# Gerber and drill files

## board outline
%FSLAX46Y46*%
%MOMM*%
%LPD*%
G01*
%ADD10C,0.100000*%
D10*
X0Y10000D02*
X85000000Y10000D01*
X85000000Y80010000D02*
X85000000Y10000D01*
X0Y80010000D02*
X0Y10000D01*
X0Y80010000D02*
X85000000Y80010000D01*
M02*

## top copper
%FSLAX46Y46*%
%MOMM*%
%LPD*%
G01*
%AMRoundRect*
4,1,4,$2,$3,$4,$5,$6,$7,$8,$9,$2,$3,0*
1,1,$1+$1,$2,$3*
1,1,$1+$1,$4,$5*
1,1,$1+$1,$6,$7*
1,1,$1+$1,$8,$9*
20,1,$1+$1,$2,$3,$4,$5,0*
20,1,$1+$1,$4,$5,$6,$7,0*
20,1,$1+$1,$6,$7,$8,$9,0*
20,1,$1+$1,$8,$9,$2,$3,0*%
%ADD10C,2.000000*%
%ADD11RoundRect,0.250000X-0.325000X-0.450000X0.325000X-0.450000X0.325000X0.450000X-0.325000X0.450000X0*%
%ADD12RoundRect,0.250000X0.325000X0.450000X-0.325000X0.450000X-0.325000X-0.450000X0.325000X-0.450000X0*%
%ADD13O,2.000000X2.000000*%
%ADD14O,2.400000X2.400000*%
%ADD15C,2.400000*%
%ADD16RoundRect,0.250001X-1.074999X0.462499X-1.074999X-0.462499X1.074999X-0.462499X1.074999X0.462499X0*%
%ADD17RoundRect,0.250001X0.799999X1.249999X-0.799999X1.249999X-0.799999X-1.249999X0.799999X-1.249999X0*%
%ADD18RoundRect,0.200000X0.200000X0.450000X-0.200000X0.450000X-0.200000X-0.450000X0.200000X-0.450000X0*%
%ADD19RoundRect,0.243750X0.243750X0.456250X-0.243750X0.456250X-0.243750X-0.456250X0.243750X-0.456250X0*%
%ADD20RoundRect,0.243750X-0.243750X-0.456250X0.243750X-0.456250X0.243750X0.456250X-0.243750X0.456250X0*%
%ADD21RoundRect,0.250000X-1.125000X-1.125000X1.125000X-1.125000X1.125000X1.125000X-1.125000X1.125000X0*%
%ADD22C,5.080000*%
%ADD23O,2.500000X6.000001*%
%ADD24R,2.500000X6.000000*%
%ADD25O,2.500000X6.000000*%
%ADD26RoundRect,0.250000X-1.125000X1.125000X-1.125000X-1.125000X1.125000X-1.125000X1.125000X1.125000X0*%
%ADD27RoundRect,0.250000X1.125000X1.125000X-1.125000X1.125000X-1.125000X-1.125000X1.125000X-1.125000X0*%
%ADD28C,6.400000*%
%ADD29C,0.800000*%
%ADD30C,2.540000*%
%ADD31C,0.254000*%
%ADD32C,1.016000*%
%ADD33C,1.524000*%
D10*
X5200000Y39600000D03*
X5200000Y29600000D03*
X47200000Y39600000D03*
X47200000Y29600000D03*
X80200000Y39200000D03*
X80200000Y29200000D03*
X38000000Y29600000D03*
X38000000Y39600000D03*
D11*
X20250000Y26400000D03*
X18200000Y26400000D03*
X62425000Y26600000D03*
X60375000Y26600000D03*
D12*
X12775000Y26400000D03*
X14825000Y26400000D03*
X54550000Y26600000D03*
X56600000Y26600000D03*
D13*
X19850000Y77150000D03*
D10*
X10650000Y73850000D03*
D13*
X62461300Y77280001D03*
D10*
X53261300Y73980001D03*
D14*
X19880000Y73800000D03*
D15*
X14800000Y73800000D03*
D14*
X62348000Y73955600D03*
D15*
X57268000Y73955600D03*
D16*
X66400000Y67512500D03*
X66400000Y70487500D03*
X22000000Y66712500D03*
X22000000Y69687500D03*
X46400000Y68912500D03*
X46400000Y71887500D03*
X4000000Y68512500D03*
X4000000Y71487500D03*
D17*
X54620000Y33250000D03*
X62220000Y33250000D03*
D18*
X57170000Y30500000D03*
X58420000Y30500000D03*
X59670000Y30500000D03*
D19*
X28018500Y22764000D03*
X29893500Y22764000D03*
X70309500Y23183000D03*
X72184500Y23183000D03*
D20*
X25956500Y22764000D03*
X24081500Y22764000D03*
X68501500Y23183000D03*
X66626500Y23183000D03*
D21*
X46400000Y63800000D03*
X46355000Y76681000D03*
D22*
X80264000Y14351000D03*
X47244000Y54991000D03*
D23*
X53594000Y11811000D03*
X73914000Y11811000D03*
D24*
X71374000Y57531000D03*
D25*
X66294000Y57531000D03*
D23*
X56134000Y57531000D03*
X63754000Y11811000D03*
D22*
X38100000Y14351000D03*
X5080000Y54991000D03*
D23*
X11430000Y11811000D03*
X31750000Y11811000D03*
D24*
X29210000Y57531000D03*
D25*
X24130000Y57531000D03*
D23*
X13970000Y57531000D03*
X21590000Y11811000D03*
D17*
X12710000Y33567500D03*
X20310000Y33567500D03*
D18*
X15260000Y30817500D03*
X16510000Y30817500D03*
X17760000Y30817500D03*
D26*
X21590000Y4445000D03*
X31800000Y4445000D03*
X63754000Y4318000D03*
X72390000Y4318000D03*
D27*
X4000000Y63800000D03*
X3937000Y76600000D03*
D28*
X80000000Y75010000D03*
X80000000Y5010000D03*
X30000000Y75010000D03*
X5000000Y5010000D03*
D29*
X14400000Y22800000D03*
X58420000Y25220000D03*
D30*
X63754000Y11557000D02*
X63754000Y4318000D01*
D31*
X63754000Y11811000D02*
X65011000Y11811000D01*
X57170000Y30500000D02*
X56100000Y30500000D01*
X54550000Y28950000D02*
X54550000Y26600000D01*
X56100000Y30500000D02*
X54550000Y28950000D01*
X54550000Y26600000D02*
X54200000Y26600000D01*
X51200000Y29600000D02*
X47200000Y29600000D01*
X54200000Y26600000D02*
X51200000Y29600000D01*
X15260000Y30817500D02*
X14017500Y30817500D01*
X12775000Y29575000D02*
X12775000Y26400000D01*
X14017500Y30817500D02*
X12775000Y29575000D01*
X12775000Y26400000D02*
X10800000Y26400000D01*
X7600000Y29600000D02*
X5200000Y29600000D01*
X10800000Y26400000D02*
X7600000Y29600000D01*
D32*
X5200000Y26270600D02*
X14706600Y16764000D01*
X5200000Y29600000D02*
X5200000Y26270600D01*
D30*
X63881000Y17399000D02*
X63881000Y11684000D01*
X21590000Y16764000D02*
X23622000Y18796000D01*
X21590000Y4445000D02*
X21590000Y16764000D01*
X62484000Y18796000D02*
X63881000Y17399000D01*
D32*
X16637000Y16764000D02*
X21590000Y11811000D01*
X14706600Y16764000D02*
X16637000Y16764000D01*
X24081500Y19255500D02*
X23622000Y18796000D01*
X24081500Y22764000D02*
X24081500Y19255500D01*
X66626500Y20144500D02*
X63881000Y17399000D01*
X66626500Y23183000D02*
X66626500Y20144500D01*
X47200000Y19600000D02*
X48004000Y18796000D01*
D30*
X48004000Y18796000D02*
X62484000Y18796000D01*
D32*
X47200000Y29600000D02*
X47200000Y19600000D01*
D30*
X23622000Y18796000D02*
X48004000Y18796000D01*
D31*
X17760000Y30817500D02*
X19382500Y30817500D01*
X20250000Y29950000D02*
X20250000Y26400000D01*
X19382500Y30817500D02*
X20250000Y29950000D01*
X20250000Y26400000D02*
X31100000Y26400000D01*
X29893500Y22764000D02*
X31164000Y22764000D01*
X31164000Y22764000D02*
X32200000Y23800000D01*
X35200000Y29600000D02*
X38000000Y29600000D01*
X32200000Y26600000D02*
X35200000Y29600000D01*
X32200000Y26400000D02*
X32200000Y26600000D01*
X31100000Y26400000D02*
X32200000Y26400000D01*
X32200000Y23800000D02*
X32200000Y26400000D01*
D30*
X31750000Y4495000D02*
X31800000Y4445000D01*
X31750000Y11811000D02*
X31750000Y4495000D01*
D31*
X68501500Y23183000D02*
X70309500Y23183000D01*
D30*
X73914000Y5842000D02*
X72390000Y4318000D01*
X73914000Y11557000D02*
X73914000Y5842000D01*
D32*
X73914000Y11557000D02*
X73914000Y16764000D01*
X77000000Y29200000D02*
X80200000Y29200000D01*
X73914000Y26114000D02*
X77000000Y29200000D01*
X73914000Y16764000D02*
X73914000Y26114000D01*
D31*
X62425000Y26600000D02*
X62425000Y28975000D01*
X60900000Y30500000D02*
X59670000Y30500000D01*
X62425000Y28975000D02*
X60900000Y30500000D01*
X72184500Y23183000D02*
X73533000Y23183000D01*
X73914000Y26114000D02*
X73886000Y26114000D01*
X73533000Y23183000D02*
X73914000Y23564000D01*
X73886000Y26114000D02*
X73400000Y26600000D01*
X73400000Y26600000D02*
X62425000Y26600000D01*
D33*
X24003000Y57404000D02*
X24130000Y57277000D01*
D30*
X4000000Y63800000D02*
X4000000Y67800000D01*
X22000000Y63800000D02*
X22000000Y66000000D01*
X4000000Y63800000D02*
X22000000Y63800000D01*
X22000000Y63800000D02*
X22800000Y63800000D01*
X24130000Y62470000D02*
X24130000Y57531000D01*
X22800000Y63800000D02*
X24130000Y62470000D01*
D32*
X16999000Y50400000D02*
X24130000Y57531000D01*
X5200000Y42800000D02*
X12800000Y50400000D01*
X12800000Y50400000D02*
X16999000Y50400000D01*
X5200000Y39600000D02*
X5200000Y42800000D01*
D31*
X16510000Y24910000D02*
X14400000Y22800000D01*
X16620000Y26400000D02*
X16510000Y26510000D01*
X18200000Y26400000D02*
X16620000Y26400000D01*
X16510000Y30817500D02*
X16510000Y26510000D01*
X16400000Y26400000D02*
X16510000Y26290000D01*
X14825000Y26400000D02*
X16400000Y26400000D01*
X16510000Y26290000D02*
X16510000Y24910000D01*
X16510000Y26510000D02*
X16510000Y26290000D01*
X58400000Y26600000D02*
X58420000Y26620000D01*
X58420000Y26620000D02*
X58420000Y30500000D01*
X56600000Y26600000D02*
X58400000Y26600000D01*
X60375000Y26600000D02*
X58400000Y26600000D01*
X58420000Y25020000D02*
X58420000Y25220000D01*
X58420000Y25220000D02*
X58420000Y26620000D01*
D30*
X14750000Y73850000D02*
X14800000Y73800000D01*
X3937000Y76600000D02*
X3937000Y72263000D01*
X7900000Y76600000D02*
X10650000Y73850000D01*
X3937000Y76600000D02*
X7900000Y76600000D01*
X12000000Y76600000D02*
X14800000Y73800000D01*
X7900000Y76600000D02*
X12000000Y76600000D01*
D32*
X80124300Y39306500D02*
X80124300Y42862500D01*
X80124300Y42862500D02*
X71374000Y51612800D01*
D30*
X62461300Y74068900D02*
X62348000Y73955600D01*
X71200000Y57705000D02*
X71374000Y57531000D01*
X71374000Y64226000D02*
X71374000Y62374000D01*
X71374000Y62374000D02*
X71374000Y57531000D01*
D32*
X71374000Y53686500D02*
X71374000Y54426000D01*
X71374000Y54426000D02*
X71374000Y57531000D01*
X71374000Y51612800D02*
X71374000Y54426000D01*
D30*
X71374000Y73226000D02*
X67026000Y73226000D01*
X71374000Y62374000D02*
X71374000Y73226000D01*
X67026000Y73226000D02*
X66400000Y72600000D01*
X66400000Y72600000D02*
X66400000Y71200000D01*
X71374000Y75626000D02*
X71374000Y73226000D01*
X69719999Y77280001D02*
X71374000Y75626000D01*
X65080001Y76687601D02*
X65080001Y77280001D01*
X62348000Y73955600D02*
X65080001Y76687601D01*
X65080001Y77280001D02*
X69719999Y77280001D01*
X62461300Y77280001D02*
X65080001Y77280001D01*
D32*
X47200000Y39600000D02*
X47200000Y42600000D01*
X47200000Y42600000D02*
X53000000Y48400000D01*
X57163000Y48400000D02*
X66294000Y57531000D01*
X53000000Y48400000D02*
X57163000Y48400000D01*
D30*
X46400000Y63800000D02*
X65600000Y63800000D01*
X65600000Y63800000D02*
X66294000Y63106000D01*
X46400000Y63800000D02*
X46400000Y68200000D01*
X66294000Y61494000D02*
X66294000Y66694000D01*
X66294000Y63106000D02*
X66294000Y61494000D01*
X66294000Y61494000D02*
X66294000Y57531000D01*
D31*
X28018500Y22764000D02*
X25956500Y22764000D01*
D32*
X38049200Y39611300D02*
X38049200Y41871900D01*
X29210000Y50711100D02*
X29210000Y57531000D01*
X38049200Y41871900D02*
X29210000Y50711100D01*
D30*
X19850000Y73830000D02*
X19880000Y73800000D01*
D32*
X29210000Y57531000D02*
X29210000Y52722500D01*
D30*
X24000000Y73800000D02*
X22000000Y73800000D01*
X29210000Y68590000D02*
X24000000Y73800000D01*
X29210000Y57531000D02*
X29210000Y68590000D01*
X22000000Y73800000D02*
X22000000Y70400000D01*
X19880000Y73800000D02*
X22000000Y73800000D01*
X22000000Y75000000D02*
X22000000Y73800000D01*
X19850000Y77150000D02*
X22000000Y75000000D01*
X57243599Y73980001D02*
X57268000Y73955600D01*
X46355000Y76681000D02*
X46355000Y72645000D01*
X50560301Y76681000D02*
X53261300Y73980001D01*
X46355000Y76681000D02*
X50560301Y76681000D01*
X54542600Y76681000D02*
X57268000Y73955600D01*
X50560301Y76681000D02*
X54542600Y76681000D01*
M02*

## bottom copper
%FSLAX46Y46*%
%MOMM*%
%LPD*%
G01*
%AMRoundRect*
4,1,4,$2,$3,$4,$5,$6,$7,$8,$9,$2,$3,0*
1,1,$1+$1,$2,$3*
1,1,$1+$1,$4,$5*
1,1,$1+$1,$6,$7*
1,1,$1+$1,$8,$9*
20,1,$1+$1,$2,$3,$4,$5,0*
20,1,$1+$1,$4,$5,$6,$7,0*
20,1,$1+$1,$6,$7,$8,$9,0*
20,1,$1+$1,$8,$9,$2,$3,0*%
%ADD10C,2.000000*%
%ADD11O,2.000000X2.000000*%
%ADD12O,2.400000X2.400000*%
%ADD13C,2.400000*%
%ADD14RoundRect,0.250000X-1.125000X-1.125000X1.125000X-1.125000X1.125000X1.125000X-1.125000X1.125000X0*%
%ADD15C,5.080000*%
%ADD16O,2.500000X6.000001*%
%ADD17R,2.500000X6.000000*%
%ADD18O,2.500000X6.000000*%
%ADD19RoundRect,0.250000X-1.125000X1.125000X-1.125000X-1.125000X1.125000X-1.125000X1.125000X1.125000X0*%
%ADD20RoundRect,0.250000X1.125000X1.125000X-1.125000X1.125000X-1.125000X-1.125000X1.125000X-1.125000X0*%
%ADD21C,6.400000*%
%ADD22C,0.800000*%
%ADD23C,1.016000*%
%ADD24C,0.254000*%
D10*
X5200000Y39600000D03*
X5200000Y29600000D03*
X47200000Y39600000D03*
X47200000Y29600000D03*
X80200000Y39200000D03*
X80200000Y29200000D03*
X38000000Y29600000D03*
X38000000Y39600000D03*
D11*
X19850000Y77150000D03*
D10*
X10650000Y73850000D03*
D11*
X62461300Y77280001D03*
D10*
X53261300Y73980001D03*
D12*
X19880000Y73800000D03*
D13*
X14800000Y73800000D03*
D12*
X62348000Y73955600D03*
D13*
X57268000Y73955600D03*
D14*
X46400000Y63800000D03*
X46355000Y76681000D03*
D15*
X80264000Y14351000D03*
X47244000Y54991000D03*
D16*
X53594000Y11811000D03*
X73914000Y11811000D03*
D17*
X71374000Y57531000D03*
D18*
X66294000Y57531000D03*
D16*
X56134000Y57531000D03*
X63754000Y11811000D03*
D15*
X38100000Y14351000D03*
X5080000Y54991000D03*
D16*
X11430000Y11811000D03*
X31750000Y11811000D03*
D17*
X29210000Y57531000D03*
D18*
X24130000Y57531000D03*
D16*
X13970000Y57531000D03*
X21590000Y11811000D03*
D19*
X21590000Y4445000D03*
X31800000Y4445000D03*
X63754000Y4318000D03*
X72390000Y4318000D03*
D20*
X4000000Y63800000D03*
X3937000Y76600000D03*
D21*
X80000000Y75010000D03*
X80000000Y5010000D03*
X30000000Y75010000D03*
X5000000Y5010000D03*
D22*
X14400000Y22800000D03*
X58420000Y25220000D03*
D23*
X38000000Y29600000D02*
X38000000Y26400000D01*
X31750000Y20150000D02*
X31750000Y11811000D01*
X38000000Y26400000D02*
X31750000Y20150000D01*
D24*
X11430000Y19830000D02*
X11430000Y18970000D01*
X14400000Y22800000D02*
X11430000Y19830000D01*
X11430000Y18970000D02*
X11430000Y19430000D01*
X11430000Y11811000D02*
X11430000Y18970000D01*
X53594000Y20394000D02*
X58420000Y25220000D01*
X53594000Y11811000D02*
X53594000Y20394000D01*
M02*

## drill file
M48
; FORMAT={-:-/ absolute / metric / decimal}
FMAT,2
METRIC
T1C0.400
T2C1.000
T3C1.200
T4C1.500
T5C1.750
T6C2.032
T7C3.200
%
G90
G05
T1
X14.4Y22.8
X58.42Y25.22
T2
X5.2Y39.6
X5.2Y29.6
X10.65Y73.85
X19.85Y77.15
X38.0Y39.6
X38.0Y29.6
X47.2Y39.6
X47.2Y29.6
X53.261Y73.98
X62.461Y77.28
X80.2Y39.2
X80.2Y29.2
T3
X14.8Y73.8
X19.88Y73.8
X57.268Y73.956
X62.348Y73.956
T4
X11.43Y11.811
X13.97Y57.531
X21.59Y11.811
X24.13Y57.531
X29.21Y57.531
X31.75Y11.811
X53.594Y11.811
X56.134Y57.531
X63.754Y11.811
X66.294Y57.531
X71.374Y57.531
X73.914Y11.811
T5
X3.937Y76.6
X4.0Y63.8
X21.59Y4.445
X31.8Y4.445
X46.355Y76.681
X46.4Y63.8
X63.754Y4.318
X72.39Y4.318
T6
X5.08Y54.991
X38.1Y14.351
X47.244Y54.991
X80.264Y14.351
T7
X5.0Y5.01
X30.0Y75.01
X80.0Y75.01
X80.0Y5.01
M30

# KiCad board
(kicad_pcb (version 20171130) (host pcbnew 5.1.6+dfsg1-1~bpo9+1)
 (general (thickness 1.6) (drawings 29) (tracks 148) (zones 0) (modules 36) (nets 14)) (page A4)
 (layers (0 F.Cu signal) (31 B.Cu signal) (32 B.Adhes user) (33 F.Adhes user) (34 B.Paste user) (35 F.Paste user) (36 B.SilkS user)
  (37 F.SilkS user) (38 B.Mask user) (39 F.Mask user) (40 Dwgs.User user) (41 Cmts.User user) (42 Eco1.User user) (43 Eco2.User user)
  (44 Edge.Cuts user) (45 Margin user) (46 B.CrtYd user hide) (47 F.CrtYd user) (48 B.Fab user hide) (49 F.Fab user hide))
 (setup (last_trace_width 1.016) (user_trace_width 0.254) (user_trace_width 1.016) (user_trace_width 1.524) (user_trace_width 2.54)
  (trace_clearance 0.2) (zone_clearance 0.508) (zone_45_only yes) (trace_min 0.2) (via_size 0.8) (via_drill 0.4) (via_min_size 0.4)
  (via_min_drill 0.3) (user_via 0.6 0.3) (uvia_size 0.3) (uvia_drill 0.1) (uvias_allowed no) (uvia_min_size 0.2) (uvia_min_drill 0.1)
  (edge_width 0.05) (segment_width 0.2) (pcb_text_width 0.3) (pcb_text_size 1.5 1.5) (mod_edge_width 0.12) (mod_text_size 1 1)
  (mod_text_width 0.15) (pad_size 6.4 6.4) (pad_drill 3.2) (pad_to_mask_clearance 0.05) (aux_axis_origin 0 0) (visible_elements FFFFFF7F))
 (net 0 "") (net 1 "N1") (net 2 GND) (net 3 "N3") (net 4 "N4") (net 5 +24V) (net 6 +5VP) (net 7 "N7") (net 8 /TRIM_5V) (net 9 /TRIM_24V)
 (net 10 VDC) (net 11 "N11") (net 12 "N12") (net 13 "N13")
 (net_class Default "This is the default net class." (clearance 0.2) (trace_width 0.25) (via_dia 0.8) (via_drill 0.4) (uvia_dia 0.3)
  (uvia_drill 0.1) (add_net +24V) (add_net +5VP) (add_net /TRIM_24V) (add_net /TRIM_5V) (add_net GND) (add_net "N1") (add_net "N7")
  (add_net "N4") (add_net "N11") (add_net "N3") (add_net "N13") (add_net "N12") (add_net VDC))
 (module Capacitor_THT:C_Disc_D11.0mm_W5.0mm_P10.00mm (layer F.Cu) (at 5.2 -29.6 90)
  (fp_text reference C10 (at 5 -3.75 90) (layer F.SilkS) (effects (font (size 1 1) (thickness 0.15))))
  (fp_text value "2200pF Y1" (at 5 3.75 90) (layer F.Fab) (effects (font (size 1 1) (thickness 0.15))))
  (pad 2 thru_hole circle (at 10 0 90) (size 2 2) (drill 1) (layers *.Cu *.Mask) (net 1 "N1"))
  (pad 1 thru_hole circle (at 0 0 90) (size 2 2) (drill 1) (layers *.Cu *.Mask) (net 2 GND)))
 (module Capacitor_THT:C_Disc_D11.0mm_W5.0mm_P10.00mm (layer F.Cu) (at 47.2 -29.6 90)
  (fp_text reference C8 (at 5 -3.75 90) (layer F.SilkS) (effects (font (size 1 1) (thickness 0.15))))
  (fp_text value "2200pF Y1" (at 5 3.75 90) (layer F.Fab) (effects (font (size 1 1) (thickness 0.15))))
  (pad 2 thru_hole circle (at 10 0 90) (size 2 2) (drill 1) (layers *.Cu *.Mask) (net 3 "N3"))
  (pad 1 thru_hole circle (at 0 0 90) (size 2 2) (drill 1) (layers *.Cu *.Mask) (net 2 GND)))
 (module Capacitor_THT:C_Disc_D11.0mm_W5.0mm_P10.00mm (layer F.Cu) (at 80.2 -29.2 90)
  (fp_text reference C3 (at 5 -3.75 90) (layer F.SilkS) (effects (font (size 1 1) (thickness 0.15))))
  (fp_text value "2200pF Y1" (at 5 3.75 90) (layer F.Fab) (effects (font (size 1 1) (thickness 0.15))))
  (pad 2 thru_hole circle (at 10 0 90) (size 2 2) (drill 1) (layers *.Cu *.Mask) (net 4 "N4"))
  (pad 1 thru_hole circle (at 0 0 90) (size 2 2) (drill 1) (layers *.Cu *.Mask) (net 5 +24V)))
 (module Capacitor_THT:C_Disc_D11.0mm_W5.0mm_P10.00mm (layer F.Cu) (at 38 -39.6 270)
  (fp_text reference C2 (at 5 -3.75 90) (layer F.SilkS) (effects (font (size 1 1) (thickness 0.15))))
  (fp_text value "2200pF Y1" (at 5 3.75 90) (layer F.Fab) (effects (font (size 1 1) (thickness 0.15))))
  (pad 2 thru_hole circle (at 10 0 270) (size 2 2) (drill 1) (layers *.Cu *.Mask) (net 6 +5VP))
  (pad 1 thru_hole circle (at 0 0 270) (size 2 2) (drill 1) (layers *.Cu *.Mask) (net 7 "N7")))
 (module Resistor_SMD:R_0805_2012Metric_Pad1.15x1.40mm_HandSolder (layer F.Cu) (at 19.225 -26.4)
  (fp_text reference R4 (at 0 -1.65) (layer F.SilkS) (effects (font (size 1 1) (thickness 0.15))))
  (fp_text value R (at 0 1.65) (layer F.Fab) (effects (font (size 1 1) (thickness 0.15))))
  (pad 2 smd roundrect (at 1.025 0) (size 1.15 1.4) (layers F.Cu F.Paste F.Mask) (roundrect_rratio 0.217391) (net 6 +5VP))
  (pad 1 smd roundrect (at -1.025 0) (size 1.15 1.4) (layers F.Cu F.Paste F.Mask) (roundrect_rratio 0.217391) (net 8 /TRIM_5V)))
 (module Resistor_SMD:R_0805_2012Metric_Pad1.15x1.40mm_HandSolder (layer F.Cu) (at 61.4 -26.6)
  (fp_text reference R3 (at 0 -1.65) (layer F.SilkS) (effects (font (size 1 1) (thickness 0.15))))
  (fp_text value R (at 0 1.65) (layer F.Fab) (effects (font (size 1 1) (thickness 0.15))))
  (pad 2 smd roundrect (at 1.025 0) (size 1.15 1.4) (layers F.Cu F.Paste F.Mask) (roundrect_rratio 0.217391) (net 5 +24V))
  (pad 1 smd roundrect (at -1.025 0) (size 1.15 1.4) (layers F.Cu F.Paste F.Mask) (roundrect_rratio 0.217391) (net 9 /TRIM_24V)))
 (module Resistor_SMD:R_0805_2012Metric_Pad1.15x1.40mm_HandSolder (layer F.Cu) (at 13.8 -26.4 180)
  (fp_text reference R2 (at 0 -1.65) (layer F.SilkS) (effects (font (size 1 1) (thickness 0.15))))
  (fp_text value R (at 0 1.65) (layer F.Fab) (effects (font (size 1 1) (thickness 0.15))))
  (pad 2 smd roundrect (at 1.025 0 180) (size 1.15 1.4) (layers F.Cu F.Paste F.Mask) (roundrect_rratio 0.217391) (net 2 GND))
  (pad 1 smd roundrect (at -1.025 0 180) (size 1.15 1.4) (layers F.Cu F.Paste F.Mask) (roundrect_rratio 0.217391) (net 8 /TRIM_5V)))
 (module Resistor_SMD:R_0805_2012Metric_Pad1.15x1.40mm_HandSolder (layer F.Cu) (at 55.575 -26.6 180)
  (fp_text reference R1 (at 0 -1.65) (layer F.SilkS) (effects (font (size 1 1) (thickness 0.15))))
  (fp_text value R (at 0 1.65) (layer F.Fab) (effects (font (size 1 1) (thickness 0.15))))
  (pad 2 smd roundrect (at 1.025 0 180) (size 1.15 1.4) (layers F.Cu F.Paste F.Mask) (roundrect_rratio 0.217391) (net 2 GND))
  (pad 1 smd roundrect (at -1.025 0 180) (size 1.15 1.4) (layers F.Cu F.Paste F.Mask) (roundrect_rratio 0.217391) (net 9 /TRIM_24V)))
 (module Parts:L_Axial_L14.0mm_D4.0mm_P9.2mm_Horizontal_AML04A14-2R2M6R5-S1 (layer F.Cu) (at 10.65 -73.85)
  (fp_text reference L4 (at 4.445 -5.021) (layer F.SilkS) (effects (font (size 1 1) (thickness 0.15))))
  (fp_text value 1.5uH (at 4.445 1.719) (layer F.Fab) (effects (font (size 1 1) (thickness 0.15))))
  (pad 2 thru_hole oval (at 9.2 -3.3) (size 2 2) (drill 1) (layers *.Cu *.Mask) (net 7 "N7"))
  (pad 1 thru_hole circle (at 0 0) (size 2 2) (drill 1) (layers *.Cu *.Mask) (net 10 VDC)))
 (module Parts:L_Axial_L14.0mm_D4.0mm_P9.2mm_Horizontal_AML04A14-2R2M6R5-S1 (layer F.Cu) (at 53.2613 -73.980001)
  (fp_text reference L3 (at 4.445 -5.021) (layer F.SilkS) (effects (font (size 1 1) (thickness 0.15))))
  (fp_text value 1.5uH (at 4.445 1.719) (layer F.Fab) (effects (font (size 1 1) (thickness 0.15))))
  (pad 2 thru_hole oval (at 9.2 -3.3) (size 2 2) (drill 1) (layers *.Cu *.Mask) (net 4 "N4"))
  (pad 1 thru_hole circle (at 0 0) (size 2 2) (drill 1) (layers *.Cu *.Mask) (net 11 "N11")))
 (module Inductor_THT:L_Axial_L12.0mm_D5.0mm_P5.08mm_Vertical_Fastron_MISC (layer F.Cu) (at 14.8 -73.8)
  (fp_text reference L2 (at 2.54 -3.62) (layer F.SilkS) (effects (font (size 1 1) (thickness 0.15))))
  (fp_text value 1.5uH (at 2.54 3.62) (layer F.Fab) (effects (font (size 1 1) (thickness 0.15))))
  (pad 2 thru_hole oval (at 5.08 0) (size 2.4 2.4) (drill 1.2) (layers *.Cu *.Mask) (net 7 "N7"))
  (pad 1 thru_hole circle (at 0 0) (size 2.4 2.4) (drill 1.2) (layers *.Cu *.Mask) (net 10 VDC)))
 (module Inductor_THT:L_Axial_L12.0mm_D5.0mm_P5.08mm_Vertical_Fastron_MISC (layer F.Cu) (at 57.268 -73.9556)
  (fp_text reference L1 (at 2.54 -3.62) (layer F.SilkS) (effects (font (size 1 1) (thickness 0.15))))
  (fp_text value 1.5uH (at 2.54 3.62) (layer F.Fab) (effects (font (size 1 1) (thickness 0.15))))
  (pad 2 thru_hole oval (at 5.08 0) (size 2.4 2.4) (drill 1.2) (layers *.Cu *.Mask) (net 4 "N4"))
  (pad 1 thru_hole circle (at 0 0) (size 2.4 2.4) (drill 1.2) (layers *.Cu *.Mask) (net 11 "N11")))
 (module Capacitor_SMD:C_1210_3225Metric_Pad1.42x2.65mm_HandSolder (layer F.Cu) (at 66.4 -69 270)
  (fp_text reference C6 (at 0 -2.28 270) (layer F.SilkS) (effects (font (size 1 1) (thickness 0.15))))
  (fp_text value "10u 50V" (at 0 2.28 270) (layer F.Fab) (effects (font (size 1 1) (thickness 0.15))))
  (pad 2 smd roundrect (at 1.4875 0 270) (size 1.425 2.65) (layers F.Cu F.Paste F.Mask) (roundrect_rratio 0.175439) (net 3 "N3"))
  (pad 1 smd roundrect (at -1.4875 0 270) (size 1.425 2.65) (layers F.Cu F.Paste F.Mask) (roundrect_rratio 0.175439) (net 4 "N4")))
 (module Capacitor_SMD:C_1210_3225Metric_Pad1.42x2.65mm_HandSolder (layer F.Cu) (at 22 -68.2 270)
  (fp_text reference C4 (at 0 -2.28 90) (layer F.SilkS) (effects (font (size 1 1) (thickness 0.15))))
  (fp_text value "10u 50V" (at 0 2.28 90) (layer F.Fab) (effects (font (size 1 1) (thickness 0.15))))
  (pad 2 smd roundrect (at 1.4875 0 270) (size 1.425 2.65) (layers F.Cu F.Paste F.Mask) (roundrect_rratio 0.175439) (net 1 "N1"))
  (pad 1 smd roundrect (at -1.4875 0 270) (size 1.425 2.65) (layers F.Cu F.Paste F.Mask) (roundrect_rratio 0.175439) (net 7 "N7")))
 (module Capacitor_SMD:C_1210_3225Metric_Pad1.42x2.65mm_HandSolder (layer F.Cu) (at 46.4 -70.4 270)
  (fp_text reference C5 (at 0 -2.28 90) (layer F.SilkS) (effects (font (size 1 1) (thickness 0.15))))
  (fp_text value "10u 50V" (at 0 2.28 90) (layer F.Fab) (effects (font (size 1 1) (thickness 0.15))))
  (pad 2 smd roundrect (at 1.4875 0 270) (size 1.425 2.65) (layers F.Cu F.Paste F.Mask) (roundrect_rratio 0.175439) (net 3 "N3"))
  (pad 1 smd roundrect (at -1.4875 0 270) (size 1.425 2.65) (layers F.Cu F.Paste F.Mask) (roundrect_rratio 0.175439) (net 11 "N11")))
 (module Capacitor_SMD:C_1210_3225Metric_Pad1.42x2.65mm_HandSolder (layer F.Cu) (at 4 -70 270)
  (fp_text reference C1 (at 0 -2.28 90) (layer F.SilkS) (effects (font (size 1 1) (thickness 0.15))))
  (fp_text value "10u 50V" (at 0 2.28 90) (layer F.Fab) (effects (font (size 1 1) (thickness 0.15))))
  (pad 2 smd roundrect (at 1.4875 0 270) (size 1.425 2.65) (layers F.Cu F.Paste F.Mask) (roundrect_rratio 0.175439) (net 1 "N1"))
  (pad 1 smd roundrect (at -1.4875 0 270) (size 1.425 2.65) (layers F.Cu F.Paste F.Mask) (roundrect_rratio 0.175439) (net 10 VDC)))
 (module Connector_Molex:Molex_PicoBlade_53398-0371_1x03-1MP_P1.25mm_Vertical (layer F.Cu) (at 58.42 -31.75 180)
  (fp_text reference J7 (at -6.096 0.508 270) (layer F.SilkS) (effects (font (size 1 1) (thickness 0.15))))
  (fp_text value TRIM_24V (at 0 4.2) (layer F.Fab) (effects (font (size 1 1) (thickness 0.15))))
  (pad MP smd roundrect (at 3.8 1.5 180) (size 2.1 3) (layers F.Cu F.Paste F.Mask) (roundrect_rratio 0.119048))
  (pad MP smd roundrect (at -3.8 1.5 180) (size 2.1 3) (layers F.Cu F.Paste F.Mask) (roundrect_rratio 0.119048))
  (pad 3 smd roundrect (at 1.25 -1.25 180) (size 0.8 1.3) (layers F.Cu F.Paste F.Mask) (roundrect_rratio 0.25) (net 2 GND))
  (pad 2 smd roundrect (at 0 -1.25 180) (size 0.8 1.3) (layers F.Cu F.Paste F.Mask) (roundrect_rratio 0.25) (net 9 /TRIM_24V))
  (pad 1 smd roundrect (at -1.25 -1.25 180) (size 0.8 1.3) (layers F.Cu F.Paste F.Mask) (roundrect_rratio 0.25) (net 5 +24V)))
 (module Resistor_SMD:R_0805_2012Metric (layer F.Cu) (at 28.956 -22.764 180)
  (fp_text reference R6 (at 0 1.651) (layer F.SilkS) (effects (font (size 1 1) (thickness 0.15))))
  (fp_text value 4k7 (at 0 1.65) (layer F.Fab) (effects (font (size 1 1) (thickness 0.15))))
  (pad 2 smd roundrect (at 0.9375 0 180) (size 0.975 1.4) (layers F.Cu F.Paste F.Mask) (roundrect_rratio 0.25) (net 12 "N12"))
  (pad 1 smd roundrect (at -0.9375 0 180) (size 0.975 1.4) (layers F.Cu F.Paste F.Mask) (roundrect_rratio 0.25) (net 6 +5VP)))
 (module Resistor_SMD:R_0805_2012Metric (layer F.Cu) (at 71.247 -23.183 180)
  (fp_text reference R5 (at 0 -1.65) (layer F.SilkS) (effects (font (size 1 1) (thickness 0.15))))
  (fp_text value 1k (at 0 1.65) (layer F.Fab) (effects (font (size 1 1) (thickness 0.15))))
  (pad 2 smd roundrect (at 0.9375 0 180) (size 0.975 1.4) (layers F.Cu F.Paste F.Mask) (roundrect_rratio 0.25) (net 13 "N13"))
  (pad 1 smd roundrect (at -0.9375 0 180) (size 0.975 1.4) (layers F.Cu F.Paste F.Mask) (roundrect_rratio 0.25) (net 5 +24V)))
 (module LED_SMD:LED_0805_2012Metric (layer F.Cu) (at 25.019 -22.764)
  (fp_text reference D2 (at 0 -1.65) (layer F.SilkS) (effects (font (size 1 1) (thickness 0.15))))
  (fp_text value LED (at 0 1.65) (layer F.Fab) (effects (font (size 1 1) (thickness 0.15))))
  (pad 2 smd roundrect (at 0.9375 0) (size 0.975 1.4) (layers F.Cu F.Paste F.Mask) (roundrect_rratio 0.25) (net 12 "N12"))
  (pad 1 smd roundrect (at -0.9375 0) (size 0.975 1.4) (layers F.Cu F.Paste F.Mask) (roundrect_rratio 0.25) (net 2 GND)))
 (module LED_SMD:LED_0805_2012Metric (layer F.Cu) (at 67.564 -23.183)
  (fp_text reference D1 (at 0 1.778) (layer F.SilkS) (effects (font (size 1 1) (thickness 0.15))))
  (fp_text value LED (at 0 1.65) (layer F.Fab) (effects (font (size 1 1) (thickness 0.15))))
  (pad 2 smd roundrect (at 0.9375 0) (size 0.975 1.4) (layers F.Cu F.Paste F.Mask) (roundrect_rratio 0.25) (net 13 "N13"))
  (pad 1 smd roundrect (at -0.9375 0) (size 0.975 1.4) (layers F.Cu F.Paste F.Mask) (roundrect_rratio 0.25) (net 2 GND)))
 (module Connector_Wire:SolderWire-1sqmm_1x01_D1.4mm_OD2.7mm (layer F.Cu) (at 46.4 -63.8)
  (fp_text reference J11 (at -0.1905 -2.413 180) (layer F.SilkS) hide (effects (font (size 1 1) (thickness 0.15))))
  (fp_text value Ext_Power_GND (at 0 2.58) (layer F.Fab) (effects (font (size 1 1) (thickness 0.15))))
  (pad 1 thru_hole roundrect (at 0 0) (size 2.75 2.75) (drill 1.75) (layers *.Cu *.Mask) (roundrect_rratio 0.090909) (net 3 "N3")))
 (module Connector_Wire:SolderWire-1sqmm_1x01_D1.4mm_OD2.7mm (layer F.Cu) (at 46.355 -76.681)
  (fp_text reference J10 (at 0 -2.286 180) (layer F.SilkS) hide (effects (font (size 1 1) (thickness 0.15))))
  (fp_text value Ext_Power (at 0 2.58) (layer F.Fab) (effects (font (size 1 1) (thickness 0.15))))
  (pad 1 thru_hole roundrect (at 0 0) (size 2.75 2.75) (drill 1.75) (layers *.Cu *.Mask) (roundrect_rratio 0.090909) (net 11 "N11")))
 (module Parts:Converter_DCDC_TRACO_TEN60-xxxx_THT (layer B.Cu) (at 71.374 -57.531 180)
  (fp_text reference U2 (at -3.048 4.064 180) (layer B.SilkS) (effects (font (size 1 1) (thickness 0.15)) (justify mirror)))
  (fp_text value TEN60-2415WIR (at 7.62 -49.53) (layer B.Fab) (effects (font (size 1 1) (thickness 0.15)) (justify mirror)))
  (pad 8 thru_hole circle (at -8.89 -43.18 90) (size 5.08 5.08) (drill 2.032) (layers *.Cu *.Mask))
  (pad 7 thru_hole circle (at 24.13 -2.54 90) (size 5.08 5.08) (drill 2.032) (layers *.Cu *.Mask))
  (pad 6 thru_hole oval (at 17.78 -45.72 90) (size 6.000001 2.5) (drill 1.5) (layers *.Cu *.Mask) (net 9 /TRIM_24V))
  (pad 4 thru_hole oval (at -2.54 -45.72 90) (size 6.000001 2.5) (drill 1.5) (layers *.Cu *.Mask) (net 5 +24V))
  (pad 1 thru_hole rect (at 0 0 90) (size 6 2.5) (drill 1.5) (layers *.Cu *.Mask) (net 4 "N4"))
  (pad 2 thru_hole oval (at 5.08 0 90) (size 6 2.5) (drill 1.5) (layers *.Cu *.Mask) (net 3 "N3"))
  (pad 3 thru_hole oval (at 15.24 0 90) (size 6.000001 2.5) (drill 1.5) (layers *.Cu *.Mask))
  (pad 5 thru_hole oval (at 7.62 -45.72 90) (size 6.000001 2.5) (drill 1.5) (layers *.Cu *.Mask) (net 2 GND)))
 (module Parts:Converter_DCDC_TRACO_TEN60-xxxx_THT (layer B.Cu) (at 29.21 -57.531 180)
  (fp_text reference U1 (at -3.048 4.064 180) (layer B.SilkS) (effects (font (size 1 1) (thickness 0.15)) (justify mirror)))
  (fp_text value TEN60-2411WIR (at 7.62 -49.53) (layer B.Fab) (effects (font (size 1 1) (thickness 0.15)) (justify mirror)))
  (pad 8 thru_hole circle (at -8.89 -43.18 90) (size 5.08 5.08) (drill 2.032) (layers *.Cu *.Mask))
  (pad 7 thru_hole circle (at 24.13 -2.54 90) (size 5.08 5.08) (drill 2.032) (layers *.Cu *.Mask))
  (pad 6 thru_hole oval (at 17.78 -45.72 90) (size 6.000001 2.5) (drill 1.5) (layers *.Cu *.Mask) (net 8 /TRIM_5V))
  (pad 4 thru_hole oval (at -2.54 -45.72 90) (size 6.000001 2.5) (drill 1.5) (layers *.Cu *.Mask) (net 6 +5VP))
  (pad 1 thru_hole rect (at 0 0 90) (size 6 2.5) (drill 1.5) (layers *.Cu *.Mask) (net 7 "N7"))
  (pad 2 thru_hole oval (at 5.08 0 90) (size 6 2.5) (drill 1.5) (layers *.Cu *.Mask) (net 1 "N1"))
  (pad 3 thru_hole oval (at 15.24 0 90) (size 6.000001 2.5) (drill 1.5) (layers *.Cu *.Mask))
  (pad 5 thru_hole oval (at 7.62 -45.72 90) (size 6.000001 2.5) (drill 1.5) (layers *.Cu *.Mask) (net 2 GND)))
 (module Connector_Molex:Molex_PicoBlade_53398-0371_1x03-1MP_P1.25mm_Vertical (layer F.Cu) (at 16.51 -32.0675 180)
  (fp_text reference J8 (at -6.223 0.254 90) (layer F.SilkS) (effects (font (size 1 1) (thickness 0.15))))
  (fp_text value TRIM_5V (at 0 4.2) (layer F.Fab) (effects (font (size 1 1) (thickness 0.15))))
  (pad MP smd roundrect (at 3.8 1.5 180) (size 2.1 3) (layers F.Cu F.Paste F.Mask) (roundrect_rratio 0.119048))
  (pad MP smd roundrect (at -3.8 1.5 180) (size 2.1 3) (layers F.Cu F.Paste F.Mask) (roundrect_rratio 0.119048))
  (pad 3 smd roundrect (at 1.25 -1.25 180) (size 0.8 1.3) (layers F.Cu F.Paste F.Mask) (roundrect_rratio 0.25) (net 2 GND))
  (pad 2 smd roundrect (at 0 -1.25 180) (size 0.8 1.3) (layers F.Cu F.Paste F.Mask) (roundrect_rratio 0.25) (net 8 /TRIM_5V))
  (pad 1 smd roundrect (at -1.25 -1.25 180) (size 0.8 1.3) (layers F.Cu F.Paste F.Mask) (roundrect_rratio 0.25) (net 6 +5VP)))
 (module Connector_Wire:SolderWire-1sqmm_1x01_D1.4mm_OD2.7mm (layer F.Cu) (at 21.59 -4.445 270)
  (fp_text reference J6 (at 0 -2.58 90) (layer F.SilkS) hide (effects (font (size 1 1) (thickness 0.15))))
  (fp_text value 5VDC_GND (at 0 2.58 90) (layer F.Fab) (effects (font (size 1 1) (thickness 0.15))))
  (pad 1 thru_hole roundrect (at 0 0 270) (size 2.75 2.75) (drill 1.75) (layers *.Cu *.Mask) (roundrect_rratio 0.090909) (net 2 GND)))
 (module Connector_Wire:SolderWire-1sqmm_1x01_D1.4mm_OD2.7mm (layer F.Cu) (at 31.8 -4.445 270)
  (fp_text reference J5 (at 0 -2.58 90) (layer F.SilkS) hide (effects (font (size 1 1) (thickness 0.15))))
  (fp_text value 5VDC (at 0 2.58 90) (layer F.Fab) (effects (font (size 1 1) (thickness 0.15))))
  (pad 1 thru_hole roundrect (at 0 0 270) (size 2.75 2.75) (drill 1.75) (layers *.Cu *.Mask) (roundrect_rratio 0.090909) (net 6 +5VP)))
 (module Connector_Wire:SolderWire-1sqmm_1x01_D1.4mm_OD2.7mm (layer F.Cu) (at 63.754 -4.318 270)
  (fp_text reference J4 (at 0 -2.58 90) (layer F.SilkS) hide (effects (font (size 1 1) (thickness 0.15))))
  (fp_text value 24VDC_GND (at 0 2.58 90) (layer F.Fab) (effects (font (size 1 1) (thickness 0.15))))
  (pad 1 thru_hole roundrect (at 0 0 270) (size 2.75 2.75) (drill 1.75) (layers *.Cu *.Mask) (roundrect_rratio 0.090909) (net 2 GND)))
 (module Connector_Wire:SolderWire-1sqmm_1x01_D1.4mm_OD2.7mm (layer F.Cu) (at 72.39 -4.318 270)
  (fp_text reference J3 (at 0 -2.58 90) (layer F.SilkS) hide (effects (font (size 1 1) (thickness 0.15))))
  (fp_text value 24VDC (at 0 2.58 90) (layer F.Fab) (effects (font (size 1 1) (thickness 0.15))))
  (pad 1 thru_hole roundrect (at 0 0 270) (size 2.75 2.75) (drill 1.75) (layers *.Cu *.Mask) (roundrect_rratio 0.090909) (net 5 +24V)))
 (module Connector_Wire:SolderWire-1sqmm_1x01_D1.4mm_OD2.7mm (layer F.Cu) (at 4 -63.8 180)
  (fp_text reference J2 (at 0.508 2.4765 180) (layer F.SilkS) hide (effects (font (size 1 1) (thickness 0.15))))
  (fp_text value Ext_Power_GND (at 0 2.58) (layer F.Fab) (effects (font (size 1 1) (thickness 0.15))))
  (pad 1 thru_hole roundrect (at 0 0 180) (size 2.75 2.75) (drill 1.75) (layers *.Cu *.Mask) (roundrect_rratio 0.090909) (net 1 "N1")))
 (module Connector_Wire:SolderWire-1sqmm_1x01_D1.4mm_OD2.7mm (layer F.Cu) (at 3.937 -76.6 180)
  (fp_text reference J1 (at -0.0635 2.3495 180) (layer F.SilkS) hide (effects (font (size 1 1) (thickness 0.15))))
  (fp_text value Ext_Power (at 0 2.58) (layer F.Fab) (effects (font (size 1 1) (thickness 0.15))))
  (pad 1 thru_hole roundrect (at 0 0 180) (size 2.75 2.75) (drill 1.75) (layers *.Cu *.Mask) (roundrect_rratio 0.090909) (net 10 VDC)))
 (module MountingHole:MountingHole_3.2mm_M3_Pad (layer F.Cu) (at 80 -75.01)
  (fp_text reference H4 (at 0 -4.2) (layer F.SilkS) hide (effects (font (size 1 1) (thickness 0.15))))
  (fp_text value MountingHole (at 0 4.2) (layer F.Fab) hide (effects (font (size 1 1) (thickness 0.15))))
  (pad 1 thru_hole circle (at 0 0) (size 6.4 6.4) (drill 3.2) (layers *.Cu *.Mask)))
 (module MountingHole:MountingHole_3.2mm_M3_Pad (layer F.Cu) (at 80 -5.01)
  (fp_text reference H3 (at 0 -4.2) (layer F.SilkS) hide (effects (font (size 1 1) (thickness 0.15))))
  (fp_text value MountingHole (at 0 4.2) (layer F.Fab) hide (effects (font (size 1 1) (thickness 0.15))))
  (pad 1 thru_hole circle (at 0 0) (size 6.4 6.4) (drill 3.2) (layers *.Cu *.Mask)))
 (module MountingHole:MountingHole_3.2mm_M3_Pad (layer F.Cu) (at 30 -75.01)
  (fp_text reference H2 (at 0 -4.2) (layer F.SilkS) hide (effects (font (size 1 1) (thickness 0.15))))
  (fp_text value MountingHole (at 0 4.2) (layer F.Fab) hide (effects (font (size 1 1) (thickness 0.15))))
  (pad 1 thru_hole circle (at 0 0) (size 6.4 6.4) (drill 3.2) (layers *.Cu *.Mask)))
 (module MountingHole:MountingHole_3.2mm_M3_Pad (layer F.Cu) (at 5 -5.01)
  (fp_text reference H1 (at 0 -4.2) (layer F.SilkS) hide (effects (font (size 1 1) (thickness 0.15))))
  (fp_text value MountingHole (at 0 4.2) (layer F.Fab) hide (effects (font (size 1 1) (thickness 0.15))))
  (pad 1 thru_hole circle (at 0 0) (size 6.4 6.4) (drill 3.2) (layers *.Cu *.Mask)))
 (gr_line (start 0 -0.01) (end 85 -0.01) (layer Edge.Cuts) (width 0.1))
 (gr_line (start 85 -80.01) (end 85 -0.01) (layer Edge.Cuts) (width 0.1))
 (gr_line (start 0 -80.01) (end 0 -0.01) (layer Edge.Cuts) (width 0.1))
 (gr_line (start 0 -80.01) (end 85 -80.01) (layer Edge.Cuts) (width 0.1))
 (segment (start 63.754 -11.557) (end 63.754 -4.318) (width 2.54) (layer F.Cu) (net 2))
 (segment (start 63.754 -11.811) (end 65.011 -11.811) (width 0.254) (layer F.Cu) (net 2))
 (segment (start 57.17 -30.5) (end 56.1 -30.5) (width 0.254) (layer F.Cu) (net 2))
 (segment (start 54.55 -28.95) (end 54.55 -26.6) (width 0.254) (layer F.Cu) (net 2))
 (segment (start 56.1 -30.5) (end 54.55 -28.95) (width 0.254) (layer F.Cu) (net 2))
 (segment (start 54.55 -26.6) (end 54.2 -26.6) (width 0.254) (layer F.Cu) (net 2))
 (segment (start 51.2 -29.6) (end 47.2 -29.6) (width 0.254) (layer F.Cu) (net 2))
 (segment (start 54.2 -26.6) (end 51.2 -29.6) (width 0.254) (layer F.Cu) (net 2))
 (segment (start 15.26 -30.8175) (end 14.0175 -30.8175) (width 0.254) (layer F.Cu) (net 2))
 (segment (start 12.775 -29.575) (end 12.775 -26.4) (width 0.254) (layer F.Cu) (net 2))
 (segment (start 14.0175 -30.8175) (end 12.775 -29.575) (width 0.254) (layer F.Cu) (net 2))
 (segment (start 12.775 -26.4) (end 10.8 -26.4) (width 0.254) (layer F.Cu) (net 2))
 (segment (start 7.6 -29.6) (end 5.2 -29.6) (width 0.254) (layer F.Cu) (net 2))
 (segment (start 10.8 -26.4) (end 7.6 -29.6) (width 0.254) (layer F.Cu) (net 2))
 (segment (start 5.2 -26.2706) (end 14.7066 -16.764) (width 1.016) (layer F.Cu) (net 2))
 (segment (start 5.2 -29.6) (end 5.2 -26.2706) (width 1.016) (layer F.Cu) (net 2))
 (segment (start 63.881 -17.399) (end 63.881 -11.684) (width 2.54) (layer F.Cu) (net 2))
 (segment (start 21.59 -16.764) (end 23.622 -18.796) (width 2.54) (layer F.Cu) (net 2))
 (segment (start 21.59 -4.445) (end 21.59 -16.764) (width 2.54) (layer F.Cu) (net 2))
 (segment (start 62.484 -18.796) (end 63.881 -17.399) (width 2.54) (layer F.Cu) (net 2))
 (segment (start 16.637 -16.764) (end 21.59 -11.811) (width 1.016) (layer F.Cu) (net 2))
 (segment (start 14.7066 -16.764) (end 16.637 -16.764) (width 1.016) (layer F.Cu) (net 2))
 (segment (start 24.0815 -19.2555) (end 23.622 -18.796) (width 1.016) (layer F.Cu) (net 2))
 (segment (start 24.0815 -22.764) (end 24.0815 -19.2555) (width 1.016) (layer F.Cu) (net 2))
 (segment (start 66.6265 -20.1445) (end 63.881 -17.399) (width 1.016) (layer F.Cu) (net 2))
 (segment (start 66.6265 -23.183) (end 66.6265 -20.1445) (width 1.016) (layer F.Cu) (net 2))
 (segment (start 47.2 -19.6) (end 48.004 -18.796) (width 1.016) (layer F.Cu) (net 2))
 (segment (start 48.004 -18.796) (end 62.484 -18.796) (width 2.54) (layer F.Cu) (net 2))
 (segment (start 47.2 -29.6) (end 47.2 -19.6) (width 1.016) (layer F.Cu) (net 2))
 (segment (start 23.622 -18.796) (end 48.004 -18.796) (width 2.54) (layer F.Cu) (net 2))
 (segment (start 17.76 -30.8175) (end 19.3825 -30.8175) (width 0.254) (layer F.Cu) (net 6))
 (segment (start 20.25 -29.95) (end 20.25 -26.4) (width 0.254) (layer F.Cu) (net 6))
 (segment (start 19.3825 -30.8175) (end 20.25 -29.95) (width 0.254) (layer F.Cu) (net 6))
 (segment (start 20.25 -26.4) (end 31.1 -26.4) (width 0.254) (layer F.Cu) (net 6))
 (segment (start 38 -29.6) (end 38 -26.4) (width 1.016) (layer B.Cu) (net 6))
 (segment (start 31.75 -20.15) (end 31.75 -11.811) (width 1.016) (layer B.Cu) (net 6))
 (segment (start 38 -26.4) (end 31.75 -20.15) (width 1.016) (layer B.Cu) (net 6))
 (segment (start 29.8935 -22.764) (end 31.164 -22.764) (width 0.254) (layer F.Cu) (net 6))
 (segment (start 31.164 -22.764) (end 32.2 -23.8) (width 0.254) (layer F.Cu) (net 6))
 (segment (start 35.2 -29.6) (end 38 -29.6) (width 0.254) (layer F.Cu) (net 6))
 (segment (start 32.2 -26.6) (end 35.2 -29.6) (width 0.254) (layer F.Cu) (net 6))
 (segment (start 32.2 -26.4) (end 32.2 -26.6) (width 0.254) (layer F.Cu) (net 6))
 (segment (start 31.1 -26.4) (end 32.2 -26.4) (width 0.254) (layer F.Cu) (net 6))
 (segment (start 32.2 -23.8) (end 32.2 -26.4) (width 0.254) (layer F.Cu) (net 6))
 (segment (start 31.75 -4.495) (end 31.8 -4.445) (width 2.54) (layer F.Cu) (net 6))
 (segment (start 31.75 -11.811) (end 31.75 -4.495) (width 2.54) (layer F.Cu) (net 6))
 (segment (start 68.5015 -23.183) (end 70.3095 -23.183) (width 0.254) (layer F.Cu) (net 13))
 (segment (start 73.914 -5.842) (end 72.39 -4.318) (width 2.54) (layer F.Cu) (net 5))
 (segment (start 73.914 -11.557) (end 73.914 -5.842) (width 2.54) (layer F.Cu) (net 5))
 (segment (start 73.914 -11.557) (end 73.914 -16.764) (width 1.016) (layer F.Cu) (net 5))
 (segment (start 77 -29.2) (end 80.2 -29.2) (width 1.016) (layer F.Cu) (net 5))
 (segment (start 73.914 -26.114) (end 77 -29.2) (width 1.016) (layer F.Cu) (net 5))
 (segment (start 73.914 -16.764) (end 73.914 -26.114) (width 1.016) (layer F.Cu) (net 5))
 (segment (start 62.425 -26.6) (end 62.425 -28.975) (width 0.254) (layer F.Cu) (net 5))
 (segment (start 60.9 -30.5) (end 59.67 -30.5) (width 0.254) (layer F.Cu) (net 5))
 (segment (start 62.425 -28.975) (end 60.9 -30.5) (width 0.254) (layer F.Cu) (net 5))
 (segment (start 72.1845 -23.183) (end 73.533 -23.183) (width 0.254) (layer F.Cu) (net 5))
 (segment (start 73.914 -26.114) (end 73.886 -26.114) (width 0.254) (layer F.Cu) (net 5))
 (segment (start 73.533 -23.183) (end 73.914 -23.564) (width 0.254) (layer F.Cu) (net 5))
 (segment (start 73.886 -26.114) (end 73.4 -26.6) (width 0.254) (layer F.Cu) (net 5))
 (segment (start 73.4 -26.6) (end 62.425 -26.6) (width 0.254) (layer F.Cu) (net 5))
 (segment (start 24.003 -57.404) (end 24.13 -57.277) (width 1.524) (layer F.Cu) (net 1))
 (segment (start 4 -63.8) (end 4 -67.8) (width 2.54) (layer F.Cu) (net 1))
 (segment (start 22 -63.8) (end 22 -66) (width 2.54) (layer F.Cu) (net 1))
 (segment (start 4 -63.8) (end 22 -63.8) (width 2.54) (layer F.Cu) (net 1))
 (segment (start 22 -63.8) (end 22.8 -63.8) (width 2.54) (layer F.Cu) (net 1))
 (segment (start 24.13 -62.47) (end 24.13 -57.531) (width 2.54) (layer F.Cu) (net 1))
 (segment (start 22.8 -63.8) (end 24.13 -62.47) (width 2.54) (layer F.Cu) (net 1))
 (segment (start 16.999 -50.4) (end 24.13 -57.531) (width 1.016) (layer F.Cu) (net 1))
 (segment (start 5.2 -42.8) (end 12.8 -50.4) (width 1.016) (layer F.Cu) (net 1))
 (segment (start 12.8 -50.4) (end 16.999 -50.4) (width 1.016) (layer F.Cu) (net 1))
 (segment (start 5.2 -39.6) (end 5.2 -42.8) (width 1.016) (layer F.Cu) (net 1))
 (via (at 14.4 -22.8) (size 0.8) (drill 0.4) (layers F.Cu B.Cu) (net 8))
 (segment (start 16.51 -24.91) (end 14.4 -22.8) (width 0.254) (layer F.Cu) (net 8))
 (segment (start 11.43 -19.83) (end 11.43 -18.97) (width 0.254) (layer B.Cu) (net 8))
 (segment (start 14.4 -22.8) (end 11.43 -19.83) (width 0.254) (layer B.Cu) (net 8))
 (segment (start 11.43 -18.97) (end 11.43 -19.43) (width 0.254) (layer B.Cu) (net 8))
 (segment (start 11.43 -11.811) (end 11.43 -18.97) (width 0.254) (layer B.Cu) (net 8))
 (segment (start 16.62 -26.4) (end 16.51 -26.51) (width 0.254) (layer F.Cu) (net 8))
 (segment (start 18.2 -26.4) (end 16.62 -26.4) (width 0.254) (layer F.Cu) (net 8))
 (segment (start 16.51 -30.8175) (end 16.51 -26.51) (width 0.254) (layer F.Cu) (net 8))
 (segment (start 16.4 -26.4) (end 16.51 -26.29) (width 0.254) (layer F.Cu) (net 8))
 (segment (start 14.825 -26.4) (end 16.4 -26.4) (width 0.254) (layer F.Cu) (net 8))
 (segment (start 16.51 -26.29) (end 16.51 -24.91) (width 0.254) (layer F.Cu) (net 8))
 (segment (start 16.51 -26.51) (end 16.51 -26.29) (width 0.254) (layer F.Cu) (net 8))
 (segment (start 58.4 -26.6) (end 58.42 -26.62) (width 0.254) (layer F.Cu) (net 9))
 (segment (start 58.42 -26.62) (end 58.42 -30.5) (width 0.254) (layer F.Cu) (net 9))
 (segment (start 56.6 -26.6) (end 58.4 -26.6) (width 0.254) (layer F.Cu) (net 9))
 (segment (start 60.375 -26.6) (end 58.4 -26.6) (width 0.254) (layer F.Cu) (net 9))
 (via (at 58.42 -25.22) (size 0.8) (drill 0.4) (layers F.Cu B.Cu) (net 9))
 (segment (start 58.42 -25.02) (end 58.42 -25.22) (width 0.254) (layer F.Cu) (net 9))
 (segment (start 53.594 -20.394) (end 58.42 -25.22) (width 0.254) (layer B.Cu) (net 9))
 (segment (start 58.42 -25.22) (end 58.42 -26.62) (width 0.254) (layer F.Cu) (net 9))
 (segment (start 53.594 -11.811) (end 53.594 -20.394) (width 0.254) (layer B.Cu) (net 9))
 (segment (start 14.75 -73.85) (end 14.8 -73.8) (width 2.54) (layer F.Cu) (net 10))
 (segment (start 3.937 -76.6) (end 3.937 -72.263) (width 2.54) (layer F.Cu) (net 10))
 (segment (start 7.9 -76.6) (end 10.65 -73.85) (width 2.54) (layer F.Cu) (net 10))
 (segment (start 3.937 -76.6) (end 7.9 -76.6) (width 2.54) (layer F.Cu) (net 10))
 (segment (start 12 -76.6) (end 14.8 -73.8) (width 2.54) (layer F.Cu) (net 10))
 (segment (start 7.9 -76.6) (end 12 -76.6) (width 2.54) (layer F.Cu) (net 10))
 (segment (start 80.1243 -39.3065) (end 80.1243 -42.8625) (width 1.016) (layer F.Cu) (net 4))
 (segment (start 80.1243 -42.8625) (end 71.374 -51.6128) (width 1.016) (layer F.Cu) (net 4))
 (segment (start 62.4613 -74.0689) (end 62.348 -73.9556) (width 2.54) (layer F.Cu) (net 4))
 (segment (start 71.2 -57.705) (end 71.374 -57.531) (width 2.54) (layer F.Cu) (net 4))
 (segment (start 71.374 -64.226) (end 71.374 -62.374) (width 2.54) (layer F.Cu) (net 4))
 (segment (start 71.374 -62.374) (end 71.374 -57.531) (width 2.54) (layer F.Cu) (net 4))
 (segment (start 71.374 -53.6865) (end 71.374 -54.426) (width 1.016) (layer F.Cu) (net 4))
 (segment (start 71.374 -54.426) (end 71.374 -57.531) (width 1.016) (layer F.Cu) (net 4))
 (segment (start 71.374 -51.6128) (end 71.374 -54.426) (width 1.016) (layer F.Cu) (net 4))
 (segment (start 71.374 -73.226) (end 67.026 -73.226) (width 2.54) (layer F.Cu) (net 4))
 (segment (start 71.374 -62.374) (end 71.374 -73.226) (width 2.54) (layer F.Cu) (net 4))
 (segment (start 67.026 -73.226) (end 66.4 -72.6) (width 2.54) (layer F.Cu) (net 4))
 (segment (start 66.4 -72.6) (end 66.4 -71.2) (width 2.54) (layer F.Cu) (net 4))
 (segment (start 71.374 -75.626) (end 71.374 -73.226) (width 2.54) (layer F.Cu) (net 4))
 (segment (start 69.719999 -77.280001) (end 71.374 -75.626) (width 2.54) (layer F.Cu) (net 4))
 (segment (start 65.080001 -76.687601) (end 65.080001 -77.280001) (width 2.54) (layer F.Cu) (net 4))
 (segment (start 62.348 -73.9556) (end 65.080001 -76.687601) (width 2.54) (layer F.Cu) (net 4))
 (segment (start 65.080001 -77.280001) (end 69.719999 -77.280001) (width 2.54) (layer F.Cu) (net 4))
 (segment (start 62.4613 -77.280001) (end 65.080001 -77.280001) (width 2.54) (layer F.Cu) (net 4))
 (segment (start 47.2 -39.6) (end 47.2 -42.6) (width 1.016) (layer F.Cu) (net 3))
 (segment (start 47.2 -42.6) (end 53 -48.4) (width 1.016) (layer F.Cu) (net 3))
 (segment (start 57.163 -48.4) (end 66.294 -57.531) (width 1.016) (layer F.Cu) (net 3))
 (segment (start 53 -48.4) (end 57.163 -48.4) (width 1.016) (layer F.Cu) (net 3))
 (segment (start 46.4 -63.8) (end 65.6 -63.8) (width 2.54) (layer F.Cu) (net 3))
 (segment (start 65.6 -63.8) (end 66.294 -63.106) (width 2.54) (layer F.Cu) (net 3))
 (segment (start 46.4 -63.8) (end 46.4 -68.2) (width 2.54) (layer F.Cu) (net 3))
 (segment (start 66.294 -61.494) (end 66.294 -66.694) (width 2.54) (layer F.Cu) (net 3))
 (segment (start 66.294 -63.106) (end 66.294 -61.494) (width 2.54) (layer F.Cu) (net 3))
 (segment (start 66.294 -61.494) (end 66.294 -57.531) (width 2.54) (layer F.Cu) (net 3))
 (segment (start 28.0185 -22.764) (end 25.9565 -22.764) (width 0.254) (layer F.Cu) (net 12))
 (segment (start 38.0492 -39.6113) (end 38.0492 -41.8719) (width 1.016) (layer F.Cu) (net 7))
 (segment (start 29.21 -50.7111) (end 29.21 -57.531) (width 1.016) (layer F.Cu) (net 7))
 (segment (start 38.0492 -41.8719) (end 29.21 -50.7111) (width 1.016) (layer F.Cu) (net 7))
 (segment (start 19.85 -73.83) (end 19.88 -73.8) (width 2.54) (layer F.Cu) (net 7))
 (segment (start 29.21 -57.531) (end 29.21 -52.7225) (width 1.016) (layer F.Cu) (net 7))
 (segment (start 24 -73.8) (end 22 -73.8) (width 2.54) (layer F.Cu) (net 7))
 (segment (start 29.21 -68.59) (end 24 -73.8) (width 2.54) (layer F.Cu) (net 7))
 (segment (start 29.21 -57.531) (end 29.21 -68.59) (width 2.54) (layer F.Cu) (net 7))
 (segment (start 22 -73.8) (end 22 -70.4) (width 2.54) (layer F.Cu) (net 7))
 (segment (start 19.88 -73.8) (end 22 -73.8) (width 2.54) (layer F.Cu) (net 7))
 (segment (start 22 -75) (end 22 -73.8) (width 2.54) (layer F.Cu) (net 7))
 (segment (start 19.85 -77.15) (end 22 -75) (width 2.54) (layer F.Cu) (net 7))
 (segment (start 57.243599 -73.980001) (end 57.268 -73.9556) (width 2.54) (layer F.Cu) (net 11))
 (segment (start 46.355 -76.681) (end 46.355 -72.645) (width 2.54) (layer F.Cu) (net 11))
 (segment (start 50.560301 -76.681) (end 53.2613 -73.980001) (width 2.54) (layer F.Cu) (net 11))
 (segment (start 46.355 -76.681) (end 50.560301 -76.681) (width 2.54) (layer F.Cu) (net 11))
 (segment (start 54.5426 -76.681) (end 57.268 -73.9556) (width 2.54) (layer F.Cu) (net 11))
 (segment (start 50.560301 -76.681) (end 54.5426 -76.681) (width 2.54) (layer F.Cu) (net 11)))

